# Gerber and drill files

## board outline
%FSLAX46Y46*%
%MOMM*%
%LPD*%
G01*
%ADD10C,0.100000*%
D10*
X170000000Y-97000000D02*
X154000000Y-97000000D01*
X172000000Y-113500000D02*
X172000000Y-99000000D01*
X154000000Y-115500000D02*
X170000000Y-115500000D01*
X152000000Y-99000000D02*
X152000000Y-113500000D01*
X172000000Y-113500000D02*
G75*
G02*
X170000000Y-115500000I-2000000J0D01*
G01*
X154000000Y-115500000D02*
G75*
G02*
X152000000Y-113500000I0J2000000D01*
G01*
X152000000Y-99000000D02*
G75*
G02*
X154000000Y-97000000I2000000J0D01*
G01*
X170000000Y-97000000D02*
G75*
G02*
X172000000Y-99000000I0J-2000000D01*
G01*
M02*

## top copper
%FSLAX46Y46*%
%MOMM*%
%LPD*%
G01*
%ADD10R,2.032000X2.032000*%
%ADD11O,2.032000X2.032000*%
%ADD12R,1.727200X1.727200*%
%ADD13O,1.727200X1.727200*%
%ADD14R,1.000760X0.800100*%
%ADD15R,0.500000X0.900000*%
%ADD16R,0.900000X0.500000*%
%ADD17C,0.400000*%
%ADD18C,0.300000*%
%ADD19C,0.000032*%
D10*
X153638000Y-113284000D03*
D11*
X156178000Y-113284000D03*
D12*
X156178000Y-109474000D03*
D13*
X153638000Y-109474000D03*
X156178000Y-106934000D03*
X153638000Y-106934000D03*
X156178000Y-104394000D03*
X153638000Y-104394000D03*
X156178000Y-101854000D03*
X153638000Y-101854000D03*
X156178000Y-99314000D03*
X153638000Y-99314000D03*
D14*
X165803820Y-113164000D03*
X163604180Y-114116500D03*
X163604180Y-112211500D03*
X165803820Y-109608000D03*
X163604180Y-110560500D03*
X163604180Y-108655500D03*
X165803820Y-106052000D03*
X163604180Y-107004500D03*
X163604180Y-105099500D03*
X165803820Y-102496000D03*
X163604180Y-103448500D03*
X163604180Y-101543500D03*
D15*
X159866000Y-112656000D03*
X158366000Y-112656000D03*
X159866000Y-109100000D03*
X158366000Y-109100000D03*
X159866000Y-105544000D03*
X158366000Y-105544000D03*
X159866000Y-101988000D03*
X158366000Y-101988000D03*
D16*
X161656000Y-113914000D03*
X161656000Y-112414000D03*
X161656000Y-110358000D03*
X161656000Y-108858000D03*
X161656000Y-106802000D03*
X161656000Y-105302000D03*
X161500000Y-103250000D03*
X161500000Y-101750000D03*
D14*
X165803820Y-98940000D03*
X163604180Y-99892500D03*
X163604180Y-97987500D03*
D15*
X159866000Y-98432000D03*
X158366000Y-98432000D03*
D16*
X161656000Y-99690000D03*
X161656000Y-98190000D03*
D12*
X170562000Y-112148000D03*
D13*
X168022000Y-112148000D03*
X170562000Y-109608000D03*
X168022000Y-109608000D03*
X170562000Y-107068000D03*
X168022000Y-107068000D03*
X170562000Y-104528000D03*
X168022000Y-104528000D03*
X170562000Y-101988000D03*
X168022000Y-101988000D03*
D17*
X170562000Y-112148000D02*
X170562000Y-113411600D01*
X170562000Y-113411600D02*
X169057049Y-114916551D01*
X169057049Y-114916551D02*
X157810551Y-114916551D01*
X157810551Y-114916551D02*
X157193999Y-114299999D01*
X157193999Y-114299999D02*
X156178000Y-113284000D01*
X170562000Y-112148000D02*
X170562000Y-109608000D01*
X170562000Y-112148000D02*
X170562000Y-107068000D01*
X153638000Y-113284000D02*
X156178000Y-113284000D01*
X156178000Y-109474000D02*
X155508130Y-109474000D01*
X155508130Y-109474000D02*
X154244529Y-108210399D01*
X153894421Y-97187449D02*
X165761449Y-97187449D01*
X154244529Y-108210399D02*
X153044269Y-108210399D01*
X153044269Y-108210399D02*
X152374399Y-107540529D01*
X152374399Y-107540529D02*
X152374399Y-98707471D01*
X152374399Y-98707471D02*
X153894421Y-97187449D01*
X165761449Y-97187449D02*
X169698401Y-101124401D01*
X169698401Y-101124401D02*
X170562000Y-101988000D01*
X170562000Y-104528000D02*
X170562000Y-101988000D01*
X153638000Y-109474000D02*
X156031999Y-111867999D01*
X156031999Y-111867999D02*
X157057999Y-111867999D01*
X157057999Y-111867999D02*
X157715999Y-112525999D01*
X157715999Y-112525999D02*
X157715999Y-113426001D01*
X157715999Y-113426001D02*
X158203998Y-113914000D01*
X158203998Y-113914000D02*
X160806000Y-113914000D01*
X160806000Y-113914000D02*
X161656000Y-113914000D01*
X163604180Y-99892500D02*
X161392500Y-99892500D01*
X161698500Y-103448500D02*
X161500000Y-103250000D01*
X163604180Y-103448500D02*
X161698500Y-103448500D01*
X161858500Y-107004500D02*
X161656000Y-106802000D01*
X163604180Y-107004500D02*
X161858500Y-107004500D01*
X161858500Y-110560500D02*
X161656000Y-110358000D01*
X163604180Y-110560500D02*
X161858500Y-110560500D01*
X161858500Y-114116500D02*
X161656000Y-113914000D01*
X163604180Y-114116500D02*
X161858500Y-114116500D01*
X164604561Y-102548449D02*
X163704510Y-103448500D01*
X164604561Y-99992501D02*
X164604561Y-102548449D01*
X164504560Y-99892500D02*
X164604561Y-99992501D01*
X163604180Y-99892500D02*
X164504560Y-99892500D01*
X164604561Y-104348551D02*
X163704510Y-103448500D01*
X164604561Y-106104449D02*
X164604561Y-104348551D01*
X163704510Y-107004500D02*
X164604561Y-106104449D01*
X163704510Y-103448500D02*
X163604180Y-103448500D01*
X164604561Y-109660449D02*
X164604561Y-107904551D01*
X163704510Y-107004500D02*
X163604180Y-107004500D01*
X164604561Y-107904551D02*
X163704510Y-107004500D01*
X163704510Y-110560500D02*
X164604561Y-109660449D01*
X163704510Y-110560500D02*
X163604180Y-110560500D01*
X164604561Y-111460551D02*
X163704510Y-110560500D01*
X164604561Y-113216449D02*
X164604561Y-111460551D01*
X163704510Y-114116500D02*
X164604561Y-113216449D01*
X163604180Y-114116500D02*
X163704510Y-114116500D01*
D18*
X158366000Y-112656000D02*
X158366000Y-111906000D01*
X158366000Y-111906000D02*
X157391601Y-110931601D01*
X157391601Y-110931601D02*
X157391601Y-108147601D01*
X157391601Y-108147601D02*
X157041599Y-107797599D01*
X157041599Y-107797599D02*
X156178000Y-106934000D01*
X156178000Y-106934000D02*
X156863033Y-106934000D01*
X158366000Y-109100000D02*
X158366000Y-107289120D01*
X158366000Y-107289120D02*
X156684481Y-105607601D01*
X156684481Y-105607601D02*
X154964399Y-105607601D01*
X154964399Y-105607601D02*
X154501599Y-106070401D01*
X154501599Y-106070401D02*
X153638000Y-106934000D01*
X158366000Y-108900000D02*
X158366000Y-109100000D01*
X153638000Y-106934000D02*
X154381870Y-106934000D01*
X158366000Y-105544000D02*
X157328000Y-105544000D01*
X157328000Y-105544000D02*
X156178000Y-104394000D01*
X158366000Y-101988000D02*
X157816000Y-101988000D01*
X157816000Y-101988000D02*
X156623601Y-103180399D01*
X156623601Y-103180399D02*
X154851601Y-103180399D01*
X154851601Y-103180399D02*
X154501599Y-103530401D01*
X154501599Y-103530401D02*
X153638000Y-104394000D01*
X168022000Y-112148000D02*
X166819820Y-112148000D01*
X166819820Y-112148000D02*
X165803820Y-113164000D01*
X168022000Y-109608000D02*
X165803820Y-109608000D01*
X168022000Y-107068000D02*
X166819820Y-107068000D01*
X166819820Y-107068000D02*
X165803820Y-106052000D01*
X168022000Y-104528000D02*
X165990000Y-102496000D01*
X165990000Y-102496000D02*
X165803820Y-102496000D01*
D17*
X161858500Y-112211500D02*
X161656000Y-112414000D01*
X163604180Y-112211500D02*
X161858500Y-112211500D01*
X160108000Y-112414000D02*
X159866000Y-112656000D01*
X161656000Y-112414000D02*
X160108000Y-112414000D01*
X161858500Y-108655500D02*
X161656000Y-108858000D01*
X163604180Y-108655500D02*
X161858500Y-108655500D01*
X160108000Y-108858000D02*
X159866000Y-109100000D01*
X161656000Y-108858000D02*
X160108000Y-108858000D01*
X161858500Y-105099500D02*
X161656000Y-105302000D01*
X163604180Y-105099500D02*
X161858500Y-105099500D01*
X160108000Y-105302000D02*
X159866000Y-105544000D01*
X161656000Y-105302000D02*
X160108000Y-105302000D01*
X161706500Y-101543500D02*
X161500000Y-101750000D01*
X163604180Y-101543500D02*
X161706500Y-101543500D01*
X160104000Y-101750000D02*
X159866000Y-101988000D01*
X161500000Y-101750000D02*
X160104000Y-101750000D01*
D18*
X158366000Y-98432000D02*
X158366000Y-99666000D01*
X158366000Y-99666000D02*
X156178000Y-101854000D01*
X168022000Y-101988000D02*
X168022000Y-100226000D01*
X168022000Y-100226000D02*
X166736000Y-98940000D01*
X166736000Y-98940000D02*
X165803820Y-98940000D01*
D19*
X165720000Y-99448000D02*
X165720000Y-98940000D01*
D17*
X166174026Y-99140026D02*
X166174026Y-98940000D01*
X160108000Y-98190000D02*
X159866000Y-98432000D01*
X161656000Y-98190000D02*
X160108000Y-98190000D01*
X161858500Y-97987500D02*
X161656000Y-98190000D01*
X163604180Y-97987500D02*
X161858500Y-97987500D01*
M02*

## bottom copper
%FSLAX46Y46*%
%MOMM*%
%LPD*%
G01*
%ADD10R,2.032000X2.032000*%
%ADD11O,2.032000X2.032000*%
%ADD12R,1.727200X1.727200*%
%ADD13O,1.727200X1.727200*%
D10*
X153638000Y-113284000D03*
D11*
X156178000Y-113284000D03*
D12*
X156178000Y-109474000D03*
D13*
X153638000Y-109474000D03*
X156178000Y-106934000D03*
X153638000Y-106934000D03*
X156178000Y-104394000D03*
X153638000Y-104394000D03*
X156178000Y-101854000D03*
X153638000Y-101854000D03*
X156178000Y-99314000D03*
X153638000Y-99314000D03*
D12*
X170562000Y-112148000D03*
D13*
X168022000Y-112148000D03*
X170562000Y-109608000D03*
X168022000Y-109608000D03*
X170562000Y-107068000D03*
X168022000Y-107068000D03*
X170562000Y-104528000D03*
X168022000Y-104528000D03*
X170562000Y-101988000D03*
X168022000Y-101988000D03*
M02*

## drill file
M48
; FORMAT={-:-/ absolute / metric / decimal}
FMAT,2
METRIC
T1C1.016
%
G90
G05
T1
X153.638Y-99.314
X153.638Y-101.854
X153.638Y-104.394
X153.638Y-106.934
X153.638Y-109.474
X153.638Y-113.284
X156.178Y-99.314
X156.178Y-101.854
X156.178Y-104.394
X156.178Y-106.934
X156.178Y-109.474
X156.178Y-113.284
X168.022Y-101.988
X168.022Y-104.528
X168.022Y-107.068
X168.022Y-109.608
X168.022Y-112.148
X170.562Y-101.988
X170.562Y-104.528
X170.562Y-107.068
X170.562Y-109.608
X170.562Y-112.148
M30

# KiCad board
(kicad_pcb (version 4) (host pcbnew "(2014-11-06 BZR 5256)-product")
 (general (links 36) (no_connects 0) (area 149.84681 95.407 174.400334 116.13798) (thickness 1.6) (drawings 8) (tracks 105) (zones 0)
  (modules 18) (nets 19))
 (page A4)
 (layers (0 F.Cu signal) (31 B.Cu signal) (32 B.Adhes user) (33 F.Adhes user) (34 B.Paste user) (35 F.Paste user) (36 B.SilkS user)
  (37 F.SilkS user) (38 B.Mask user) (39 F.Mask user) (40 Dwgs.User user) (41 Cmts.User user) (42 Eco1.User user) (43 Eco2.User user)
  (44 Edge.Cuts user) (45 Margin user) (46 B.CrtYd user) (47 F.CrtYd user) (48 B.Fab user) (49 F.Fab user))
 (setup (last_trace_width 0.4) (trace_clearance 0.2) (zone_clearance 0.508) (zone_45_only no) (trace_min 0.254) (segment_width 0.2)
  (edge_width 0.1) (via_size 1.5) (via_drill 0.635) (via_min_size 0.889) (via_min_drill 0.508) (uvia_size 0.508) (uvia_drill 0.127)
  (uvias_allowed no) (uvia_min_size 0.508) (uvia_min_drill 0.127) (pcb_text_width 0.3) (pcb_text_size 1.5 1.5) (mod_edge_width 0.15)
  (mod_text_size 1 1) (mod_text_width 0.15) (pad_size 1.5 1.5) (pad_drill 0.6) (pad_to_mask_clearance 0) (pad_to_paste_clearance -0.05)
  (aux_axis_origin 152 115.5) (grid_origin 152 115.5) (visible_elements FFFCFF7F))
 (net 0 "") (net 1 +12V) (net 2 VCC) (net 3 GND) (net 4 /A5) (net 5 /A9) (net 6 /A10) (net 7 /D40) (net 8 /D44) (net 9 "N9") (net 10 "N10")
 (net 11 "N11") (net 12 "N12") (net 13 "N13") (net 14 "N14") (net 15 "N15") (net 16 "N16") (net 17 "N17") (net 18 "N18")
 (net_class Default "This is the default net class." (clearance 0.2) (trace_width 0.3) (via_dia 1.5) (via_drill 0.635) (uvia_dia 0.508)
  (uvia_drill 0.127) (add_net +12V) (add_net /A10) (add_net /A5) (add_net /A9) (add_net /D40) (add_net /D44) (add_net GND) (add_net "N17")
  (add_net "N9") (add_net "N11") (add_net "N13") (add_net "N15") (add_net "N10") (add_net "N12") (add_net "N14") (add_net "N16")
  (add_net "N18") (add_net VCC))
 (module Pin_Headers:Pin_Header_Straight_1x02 (layer F.Cu) (at 154.908 113.284)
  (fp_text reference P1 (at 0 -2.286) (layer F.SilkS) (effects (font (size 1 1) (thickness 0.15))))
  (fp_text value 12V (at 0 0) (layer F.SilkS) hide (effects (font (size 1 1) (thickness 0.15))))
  (pad 1 thru_hole rect (at -1.27 0) (size 2.032 2.032) (drill 1.016) (layers *.Cu *.Mask F.SilkS) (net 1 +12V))
  (pad 2 thru_hole oval (at 1.27 0) (size 2.032 2.032) (drill 1.016) (layers *.Cu *.Mask F.SilkS) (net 1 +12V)))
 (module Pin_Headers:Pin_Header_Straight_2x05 (layer F.Cu) (at 154.908 104.394 90)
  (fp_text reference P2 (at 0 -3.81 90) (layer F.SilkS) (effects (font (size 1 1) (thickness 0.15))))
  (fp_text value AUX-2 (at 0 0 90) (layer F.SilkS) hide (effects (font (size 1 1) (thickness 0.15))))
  (pad 1 thru_hole rect (at -5.08 1.27 90) (size 1.7272 1.7272) (drill 1.016) (layers *.Cu *.Mask F.SilkS) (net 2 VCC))
  (pad 2 thru_hole oval (at -5.08 -1.27 90) (size 1.7272 1.7272) (drill 1.016) (layers *.Cu *.Mask F.SilkS) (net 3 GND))
  (pad 3 thru_hole oval (at -2.54 1.27 90) (size 1.7272 1.7272) (drill 1.016) (layers *.Cu *.Mask F.SilkS) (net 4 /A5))
  (pad 4 thru_hole oval (at -2.54 -1.27 90) (size 1.7272 1.7272) (drill 1.016) (layers *.Cu *.Mask F.SilkS) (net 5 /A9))
  (pad 5 thru_hole oval (at 0 1.27 90) (size 1.7272 1.7272) (drill 1.016) (layers *.Cu *.Mask F.SilkS) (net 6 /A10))
  (pad 6 thru_hole oval (at 0 -1.27 90) (size 1.7272 1.7272) (drill 1.016) (layers *.Cu *.Mask F.SilkS) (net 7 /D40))
  (pad 7 thru_hole oval (at 2.54 1.27 90) (size 1.7272 1.7272) (drill 1.016) (layers *.Cu *.Mask F.SilkS) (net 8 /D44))
  (pad 8 thru_hole oval (at 2.54 -1.27 90) (size 1.7272 1.7272) (drill 1.016) (layers *.Cu *.Mask F.SilkS))
  (pad 9 thru_hole oval (at 5.08 1.27 90) (size 1.7272 1.7272) (drill 1.016) (layers *.Cu *.Mask F.SilkS))
  (pad 10 thru_hole oval (at 5.08 -1.27 90) (size 1.7272 1.7272) (drill 1.016) (layers *.Cu *.Mask F.SilkS)))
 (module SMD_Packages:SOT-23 (layer F.Cu) (at 164.704 113.164 270)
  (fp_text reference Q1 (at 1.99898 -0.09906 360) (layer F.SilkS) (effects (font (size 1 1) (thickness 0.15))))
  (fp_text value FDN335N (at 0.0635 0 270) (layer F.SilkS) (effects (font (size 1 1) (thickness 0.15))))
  (pad 3 smd rect (at 0 -1.09982 270) (size 0.8001 1.00076) (layers F.Cu F.Paste F.Mask) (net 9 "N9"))
  (pad 2 smd rect (at 0.9525 1.09982 270) (size 0.8001 1.00076) (layers F.Cu F.Paste F.Mask) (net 3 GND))
  (pad 1 smd rect (at -0.9525 1.09982 270) (size 0.8001 1.00076) (layers F.Cu F.Paste F.Mask) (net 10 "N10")))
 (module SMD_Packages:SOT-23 (layer F.Cu) (at 164.704 109.608 270)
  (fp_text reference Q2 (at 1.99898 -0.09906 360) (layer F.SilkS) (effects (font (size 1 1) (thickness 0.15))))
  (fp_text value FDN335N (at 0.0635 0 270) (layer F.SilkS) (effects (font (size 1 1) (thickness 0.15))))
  (pad 3 smd rect (at 0 -1.09982 270) (size 0.8001 1.00076) (layers F.Cu F.Paste F.Mask) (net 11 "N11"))
  (pad 2 smd rect (at 0.9525 1.09982 270) (size 0.8001 1.00076) (layers F.Cu F.Paste F.Mask) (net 3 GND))
  (pad 1 smd rect (at -0.9525 1.09982 270) (size 0.8001 1.00076) (layers F.Cu F.Paste F.Mask) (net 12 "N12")))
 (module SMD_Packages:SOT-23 (layer F.Cu) (at 164.704 106.052 270)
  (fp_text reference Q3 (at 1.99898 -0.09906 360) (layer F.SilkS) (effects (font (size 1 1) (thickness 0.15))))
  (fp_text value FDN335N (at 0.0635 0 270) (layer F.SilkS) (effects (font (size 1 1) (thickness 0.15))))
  (pad 3 smd rect (at 0 -1.09982 270) (size 0.8001 1.00076) (layers F.Cu F.Paste F.Mask) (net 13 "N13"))
  (pad 2 smd rect (at 0.9525 1.09982 270) (size 0.8001 1.00076) (layers F.Cu F.Paste F.Mask) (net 3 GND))
  (pad 1 smd rect (at -0.9525 1.09982 270) (size 0.8001 1.00076) (layers F.Cu F.Paste F.Mask) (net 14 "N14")))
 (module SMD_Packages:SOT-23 (layer F.Cu) (at 164.704 102.496 270)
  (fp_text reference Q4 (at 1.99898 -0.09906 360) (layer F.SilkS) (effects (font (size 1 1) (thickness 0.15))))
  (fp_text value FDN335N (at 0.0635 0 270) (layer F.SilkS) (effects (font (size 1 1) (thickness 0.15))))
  (pad 3 smd rect (at 0 -1.09982 270) (size 0.8001 1.00076) (layers F.Cu F.Paste F.Mask) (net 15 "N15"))
  (pad 2 smd rect (at 0.9525 1.09982 270) (size 0.8001 1.00076) (layers F.Cu F.Paste F.Mask) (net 3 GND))
  (pad 1 smd rect (at -0.9525 1.09982 270) (size 0.8001 1.00076) (layers F.Cu F.Paste F.Mask) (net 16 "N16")))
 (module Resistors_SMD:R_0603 (layer F.Cu) (at 159.116 112.656 180)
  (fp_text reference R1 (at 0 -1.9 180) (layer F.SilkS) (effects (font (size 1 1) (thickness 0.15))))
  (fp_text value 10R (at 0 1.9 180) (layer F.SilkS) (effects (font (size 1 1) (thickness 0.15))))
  (pad 1 smd rect (at -0.75 0 180) (size 0.5 0.9) (layers F.Cu F.Paste F.Mask) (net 10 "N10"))
  (pad 2 smd rect (at 0.75 0 180) (size 0.5 0.9) (layers F.Cu F.Paste F.Mask) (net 4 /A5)))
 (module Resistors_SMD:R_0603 (layer F.Cu) (at 159.116 109.1 180)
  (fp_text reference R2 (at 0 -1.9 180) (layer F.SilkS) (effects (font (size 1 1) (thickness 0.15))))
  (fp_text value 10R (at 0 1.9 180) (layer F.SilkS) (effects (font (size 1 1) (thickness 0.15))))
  (pad 1 smd rect (at -0.75 0 180) (size 0.5 0.9) (layers F.Cu F.Paste F.Mask) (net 12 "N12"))
  (pad 2 smd rect (at 0.75 0 180) (size 0.5 0.9) (layers F.Cu F.Paste F.Mask) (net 5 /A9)))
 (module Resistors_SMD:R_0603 (layer F.Cu) (at 159.116 105.544 180)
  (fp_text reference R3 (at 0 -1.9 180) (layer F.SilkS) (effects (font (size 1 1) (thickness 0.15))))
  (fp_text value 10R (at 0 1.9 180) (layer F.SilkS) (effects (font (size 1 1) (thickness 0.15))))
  (pad 1 smd rect (at -0.75 0 180) (size 0.5 0.9) (layers F.Cu F.Paste F.Mask) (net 14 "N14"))
  (pad 2 smd rect (at 0.75 0 180) (size 0.5 0.9) (layers F.Cu F.Paste F.Mask) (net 6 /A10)))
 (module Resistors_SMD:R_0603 (layer F.Cu) (at 159.116 101.988 180)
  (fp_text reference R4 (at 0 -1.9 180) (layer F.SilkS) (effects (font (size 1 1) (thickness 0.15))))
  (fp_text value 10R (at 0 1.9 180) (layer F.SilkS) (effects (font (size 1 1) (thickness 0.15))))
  (pad 1 smd rect (at -0.75 0 180) (size 0.5 0.9) (layers F.Cu F.Paste F.Mask) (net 16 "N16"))
  (pad 2 smd rect (at 0.75 0 180) (size 0.5 0.9) (layers F.Cu F.Paste F.Mask) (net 7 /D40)))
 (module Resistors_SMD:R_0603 (layer F.Cu) (at 161.656 113.164 90)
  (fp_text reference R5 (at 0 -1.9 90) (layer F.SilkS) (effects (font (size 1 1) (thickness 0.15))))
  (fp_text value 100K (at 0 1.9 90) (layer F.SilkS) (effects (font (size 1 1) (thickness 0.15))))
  (pad 1 smd rect (at -0.75 0 90) (size 0.5 0.9) (layers F.Cu F.Paste F.Mask) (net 3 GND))
  (pad 2 smd rect (at 0.75 0 90) (size 0.5 0.9) (layers F.Cu F.Paste F.Mask) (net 10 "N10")))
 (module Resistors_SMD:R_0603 (layer F.Cu) (at 161.656 109.608 90)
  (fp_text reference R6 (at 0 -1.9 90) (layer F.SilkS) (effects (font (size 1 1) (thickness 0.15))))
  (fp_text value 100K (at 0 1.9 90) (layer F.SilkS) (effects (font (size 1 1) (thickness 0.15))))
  (pad 1 smd rect (at -0.75 0 90) (size 0.5 0.9) (layers F.Cu F.Paste F.Mask) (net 3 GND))
  (pad 2 smd rect (at 0.75 0 90) (size 0.5 0.9) (layers F.Cu F.Paste F.Mask) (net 12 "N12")))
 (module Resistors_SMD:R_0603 (layer F.Cu) (at 161.656 106.052 90)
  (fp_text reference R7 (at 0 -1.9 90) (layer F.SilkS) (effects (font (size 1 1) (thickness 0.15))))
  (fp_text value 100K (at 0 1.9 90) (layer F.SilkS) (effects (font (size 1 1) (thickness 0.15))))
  (pad 1 smd rect (at -0.75 0 90) (size 0.5 0.9) (layers F.Cu F.Paste F.Mask) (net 3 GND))
  (pad 2 smd rect (at 0.75 0 90) (size 0.5 0.9) (layers F.Cu F.Paste F.Mask) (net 14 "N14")))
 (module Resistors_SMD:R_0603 (layer F.Cu) (at 161.5 102.5 90)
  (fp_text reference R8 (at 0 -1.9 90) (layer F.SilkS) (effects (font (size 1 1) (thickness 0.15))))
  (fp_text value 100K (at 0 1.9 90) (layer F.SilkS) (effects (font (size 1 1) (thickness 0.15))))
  (pad 1 smd rect (at -0.75 0 90) (size 0.5 0.9) (layers F.Cu F.Paste F.Mask) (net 3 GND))
  (pad 2 smd rect (at 0.75 0 90) (size 0.5 0.9) (layers F.Cu F.Paste F.Mask) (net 16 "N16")))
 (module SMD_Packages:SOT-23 (layer F.Cu) (at 164.704 98.94 270)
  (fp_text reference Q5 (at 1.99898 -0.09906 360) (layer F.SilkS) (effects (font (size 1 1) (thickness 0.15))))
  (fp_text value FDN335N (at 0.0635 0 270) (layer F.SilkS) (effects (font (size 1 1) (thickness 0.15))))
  (pad 3 smd rect (at 0 -1.09982 270) (size 0.8001 1.00076) (layers F.Cu F.Paste F.Mask) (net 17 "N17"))
  (pad 2 smd rect (at 0.9525 1.09982 270) (size 0.8001 1.00076) (layers F.Cu F.Paste F.Mask) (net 3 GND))
  (pad 1 smd rect (at -0.9525 1.09982 270) (size 0.8001 1.00076) (layers F.Cu F.Paste F.Mask) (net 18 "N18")))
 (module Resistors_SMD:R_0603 (layer F.Cu) (at 159.116 98.432 180)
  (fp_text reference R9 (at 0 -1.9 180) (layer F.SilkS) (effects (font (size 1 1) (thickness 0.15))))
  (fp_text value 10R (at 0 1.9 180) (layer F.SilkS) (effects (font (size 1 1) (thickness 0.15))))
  (pad 1 smd rect (at -0.75 0 180) (size 0.5 0.9) (layers F.Cu F.Paste F.Mask) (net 18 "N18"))
  (pad 2 smd rect (at 0.75 0 180) (size 0.5 0.9) (layers F.Cu F.Paste F.Mask) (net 8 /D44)))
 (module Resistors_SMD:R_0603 (layer F.Cu) (at 161.656 98.94 90)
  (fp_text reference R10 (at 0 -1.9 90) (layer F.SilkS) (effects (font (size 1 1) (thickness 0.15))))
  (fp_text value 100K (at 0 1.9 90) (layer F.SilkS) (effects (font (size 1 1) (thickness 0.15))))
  (pad 1 smd rect (at -0.75 0 90) (size 0.5 0.9) (layers F.Cu F.Paste F.Mask) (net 3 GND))
  (pad 2 smd rect (at 0.75 0 90) (size 0.5 0.9) (layers F.Cu F.Paste F.Mask) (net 18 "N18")))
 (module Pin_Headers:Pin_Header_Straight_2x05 (layer F.Cu) (at 169.292 107.068 90)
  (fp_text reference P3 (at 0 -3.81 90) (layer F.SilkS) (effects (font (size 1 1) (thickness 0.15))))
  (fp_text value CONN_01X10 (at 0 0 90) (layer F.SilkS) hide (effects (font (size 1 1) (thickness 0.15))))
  (pad 1 thru_hole rect (at -5.08 1.27 90) (size 1.7272 1.7272) (drill 1.016) (layers *.Cu *.Mask F.SilkS) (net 1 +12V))
  (pad 2 thru_hole oval (at -5.08 -1.27 90) (size 1.7272 1.7272) (drill 1.016) (layers *.Cu *.Mask F.SilkS) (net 9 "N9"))
  (pad 3 thru_hole oval (at -2.54 1.27 90) (size 1.7272 1.7272) (drill 1.016) (layers *.Cu *.Mask F.SilkS) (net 1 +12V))
  (pad 4 thru_hole oval (at -2.54 -1.27 90) (size 1.7272 1.7272) (drill 1.016) (layers *.Cu *.Mask F.SilkS) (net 11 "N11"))
  (pad 5 thru_hole oval (at 0 1.27 90) (size 1.7272 1.7272) (drill 1.016) (layers *.Cu *.Mask F.SilkS) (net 1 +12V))
  (pad 6 thru_hole oval (at 0 -1.27 90) (size 1.7272 1.7272) (drill 1.016) (layers *.Cu *.Mask F.SilkS) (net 13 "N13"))
  (pad 7 thru_hole oval (at 2.54 1.27 90) (size 1.7272 1.7272) (drill 1.016) (layers *.Cu *.Mask F.SilkS) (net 2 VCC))
  (pad 8 thru_hole oval (at 2.54 -1.27 90) (size 1.7272 1.7272) (drill 1.016) (layers *.Cu *.Mask F.SilkS) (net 15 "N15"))
  (pad 9 thru_hole oval (at 5.08 1.27 90) (size 1.7272 1.7272) (drill 1.016) (layers *.Cu *.Mask F.SilkS) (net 2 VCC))
  (pad 10 thru_hole oval (at 5.08 -1.27 90) (size 1.7272 1.7272) (drill 1.016) (layers *.Cu *.Mask F.SilkS) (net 17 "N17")))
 (gr_line (start 170 97) (end 154 97) (angle 90) (layer Edge.Cuts) (width 0.1))
 (gr_line (start 172 113.5) (end 172 99) (angle 90) (layer Edge.Cuts) (width 0.1))
 (gr_line (start 154 115.5) (end 170 115.5) (angle 90) (layer Edge.Cuts) (width 0.1))
 (gr_line (start 152 99) (end 152 113.5) (angle 90) (layer Edge.Cuts) (width 0.1))
 (gr_arc (start 170 113.5) (end 172 113.5) (angle 90) (layer Edge.Cuts) (width 0.1))
 (gr_arc (start 154 113.5) (end 154 115.5) (angle 90) (layer Edge.Cuts) (width 0.1))
 (gr_arc (start 154 99) (end 152 99) (angle 90) (layer Edge.Cuts) (width 0.1))
 (gr_arc (start 170 99) (end 170 97) (angle 90) (layer Edge.Cuts) (width 0.1))
 (segment (start 170.562 112.148) (end 170.562 113.4116) (width 0.4) (layer F.Cu) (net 1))
 (segment (start 170.562 113.4116) (end 169.057049 114.916551) (width 0.4) (layer F.Cu) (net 1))
 (segment (start 169.057049 114.916551) (end 157.810551 114.916551) (width 0.4) (layer F.Cu) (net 1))
 (segment (start 157.810551 114.916551) (end 157.193999 114.299999) (width 0.4) (layer F.Cu) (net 1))
 (segment (start 157.193999 114.299999) (end 156.178 113.284) (width 0.4) (layer F.Cu) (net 1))
 (segment (start 170.562 112.148) (end 170.562 109.608) (width 0.4) (layer F.Cu) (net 1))
 (segment (start 170.562 112.148) (end 170.562 107.068) (width 0.4) (layer F.Cu) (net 1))
 (segment (start 153.638 113.284) (end 156.178 113.284) (width 0.4) (layer F.Cu) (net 1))
 (segment (start 156.178 109.474) (end 155.50813 109.474) (width 0.4) (layer F.Cu) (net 2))
 (segment (start 155.50813 109.474) (end 154.244529 108.210399) (width 0.4) (layer F.Cu) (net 2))
 (segment (start 153.894421 97.187449) (end 165.761449 97.187449) (width 0.4) (layer F.Cu) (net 2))
 (segment (start 154.244529 108.210399) (end 153.044269 108.210399) (width 0.4) (layer F.Cu) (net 2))
 (segment (start 153.044269 108.210399) (end 152.374399 107.540529) (width 0.4) (layer F.Cu) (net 2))
 (segment (start 152.374399 107.540529) (end 152.374399 98.707471) (width 0.4) (layer F.Cu) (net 2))
 (segment (start 152.374399 98.707471) (end 153.894421 97.187449) (width 0.4) (layer F.Cu) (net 2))
 (segment (start 165.761449 97.187449) (end 169.698401 101.124401) (width 0.4) (layer F.Cu) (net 2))
 (segment (start 169.698401 101.124401) (end 170.562 101.988) (width 0.4) (layer F.Cu) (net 2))
 (segment (start 170.562 104.528) (end 170.562 101.988) (width 0.4) (layer F.Cu) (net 2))
 (segment (start 153.638 109.474) (end 156.031999 111.867999) (width 0.4) (layer F.Cu) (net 3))
 (segment (start 156.031999 111.867999) (end 157.057999 111.867999) (width 0.4) (layer F.Cu) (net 3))
 (segment (start 157.057999 111.867999) (end 157.715999 112.525999) (width 0.4) (layer F.Cu) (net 3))
 (segment (start 157.715999 112.525999) (end 157.715999 113.426001) (width 0.4) (layer F.Cu) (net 3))
 (segment (start 157.715999 113.426001) (end 158.203998 113.914) (width 0.4) (layer F.Cu) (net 3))
 (segment (start 158.203998 113.914) (end 160.806 113.914) (width 0.4) (layer F.Cu) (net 3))
 (segment (start 160.806 113.914) (end 161.656 113.914) (width 0.4) (layer F.Cu) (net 3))
 (segment (start 163.60418 99.8925) (end 161.3925 99.8925) (width 0.4) (layer F.Cu) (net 3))
 (segment (start 161.6985 103.4485) (end 161.5 103.25) (width 0.4) (layer F.Cu) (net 3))
 (segment (start 163.60418 103.4485) (end 161.6985 103.4485) (width 0.4) (layer F.Cu) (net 3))
 (segment (start 161.8585 107.0045) (end 161.656 106.802) (width 0.4) (layer F.Cu) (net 3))
 (segment (start 163.60418 107.0045) (end 161.8585 107.0045) (width 0.4) (layer F.Cu) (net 3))
 (segment (start 161.8585 110.5605) (end 161.656 110.358) (width 0.4) (layer F.Cu) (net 3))
 (segment (start 163.60418 110.5605) (end 161.8585 110.5605) (width 0.4) (layer F.Cu) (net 3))
 (segment (start 161.8585 114.1165) (end 161.656 113.914) (width 0.4) (layer F.Cu) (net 3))
 (segment (start 163.60418 114.1165) (end 161.8585 114.1165) (width 0.4) (layer F.Cu) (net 3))
 (segment (start 164.604561 102.548449) (end 163.70451 103.4485) (width 0.4) (layer F.Cu) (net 3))
 (segment (start 164.604561 99.992501) (end 164.604561 102.548449) (width 0.4) (layer F.Cu) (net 3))
 (segment (start 164.50456 99.8925) (end 164.604561 99.992501) (width 0.4) (layer F.Cu) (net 3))
 (segment (start 163.60418 99.8925) (end 164.50456 99.8925) (width 0.4) (layer F.Cu) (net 3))
 (segment (start 164.604561 104.348551) (end 163.70451 103.4485) (width 0.4) (layer F.Cu) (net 3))
 (segment (start 164.604561 106.104449) (end 164.604561 104.348551) (width 0.4) (layer F.Cu) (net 3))
 (segment (start 163.70451 107.0045) (end 164.604561 106.104449) (width 0.4) (layer F.Cu) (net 3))
 (segment (start 163.70451 103.4485) (end 163.60418 103.4485) (width 0.4) (layer F.Cu) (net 3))
 (segment (start 164.604561 109.660449) (end 164.604561 107.904551) (width 0.4) (layer F.Cu) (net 3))
 (segment (start 163.70451 107.0045) (end 163.60418 107.0045) (width 0.4) (layer F.Cu) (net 3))
 (segment (start 164.604561 107.904551) (end 163.70451 107.0045) (width 0.4) (layer F.Cu) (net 3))
 (segment (start 163.70451 110.5605) (end 164.604561 109.660449) (width 0.4) (layer F.Cu) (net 3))
 (segment (start 163.70451 110.5605) (end 163.60418 110.5605) (width 0.4) (layer F.Cu) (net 3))
 (segment (start 164.604561 111.460551) (end 163.70451 110.5605) (width 0.4) (layer F.Cu) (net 3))
 (segment (start 164.604561 113.216449) (end 164.604561 111.460551) (width 0.4) (layer F.Cu) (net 3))
 (segment (start 163.70451 114.1165) (end 164.604561 113.216449) (width 0.4) (layer F.Cu) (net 3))
 (segment (start 163.60418 114.1165) (end 163.70451 114.1165) (width 0.4) (layer F.Cu) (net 3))
 (segment (start 158.366 112.656) (end 158.366 111.906) (width 0.3) (layer F.Cu) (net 4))
 (segment (start 158.366 111.906) (end 157.391601 110.931601) (width 0.3) (layer F.Cu) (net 4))
 (segment (start 157.391601 110.931601) (end 157.391601 108.147601) (width 0.3) (layer F.Cu) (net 4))
 (segment (start 157.391601 108.147601) (end 157.041599 107.797599) (width 0.3) (layer F.Cu) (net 4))
 (segment (start 157.041599 107.797599) (end 156.178 106.934) (width 0.3) (layer F.Cu) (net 4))
 (segment (start 156.178 106.934) (end 156.863033 106.934) (width 0.3) (layer F.Cu) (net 4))
 (segment (start 158.366 109.1) (end 158.366 107.28912) (width 0.3) (layer F.Cu) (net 5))
 (segment (start 158.366 107.28912) (end 156.684481 105.607601) (width 0.3) (layer F.Cu) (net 5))
 (segment (start 156.684481 105.607601) (end 154.964399 105.607601) (width 0.3) (layer F.Cu) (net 5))
 (segment (start 154.964399 105.607601) (end 154.501599 106.070401) (width 0.3) (layer F.Cu) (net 5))
 (segment (start 154.501599 106.070401) (end 153.638 106.934) (width 0.3) (layer F.Cu) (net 5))
 (segment (start 158.366 108.9) (end 158.366 109.1) (width 0.3) (layer F.Cu) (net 5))
 (segment (start 153.638 106.934) (end 154.38187 106.934) (width 0.3) (layer F.Cu) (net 5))
 (segment (start 158.366 105.544) (end 157.328 105.544) (width 0.3) (layer F.Cu) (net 6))
 (segment (start 157.328 105.544) (end 156.178 104.394) (width 0.3) (layer F.Cu) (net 6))
 (segment (start 158.366 101.988) (end 157.816 101.988) (width 0.3) (layer F.Cu) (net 7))
 (segment (start 157.816 101.988) (end 156.623601 103.180399) (width 0.3) (layer F.Cu) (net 7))
 (segment (start 156.623601 103.180399) (end 154.851601 103.180399) (width 0.3) (layer F.Cu) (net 7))
 (segment (start 154.851601 103.180399) (end 154.501599 103.530401) (width 0.3) (layer F.Cu) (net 7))
 (segment (start 154.501599 103.530401) (end 153.638 104.394) (width 0.3) (layer F.Cu) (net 7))
 (segment (start 168.022 112.148) (end 166.81982 112.148) (width 0.3) (layer F.Cu) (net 9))
 (segment (start 166.81982 112.148) (end 165.80382 113.164) (width 0.3) (layer F.Cu) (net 9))
 (segment (start 168.022 109.608) (end 165.80382 109.608) (width 0.3) (layer F.Cu) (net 11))
 (segment (start 168.022 107.068) (end 166.81982 107.068) (width 0.3) (layer F.Cu) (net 13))
 (segment (start 166.81982 107.068) (end 165.80382 106.052) (width 0.3) (layer F.Cu) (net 13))
 (segment (start 168.022 104.528) (end 165.99 102.496) (width 0.3) (layer F.Cu) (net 15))
 (segment (start 165.99 102.496) (end 165.80382 102.496) (width 0.3) (layer F.Cu) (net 15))
 (segment (start 161.8585 112.2115) (end 161.656 112.414) (width 0.4) (layer F.Cu) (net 10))
 (segment (start 163.60418 112.2115) (end 161.8585 112.2115) (width 0.4) (layer F.Cu) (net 10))
 (segment (start 160.108 112.414) (end 159.866 112.656) (width 0.4) (layer F.Cu) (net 10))
 (segment (start 161.656 112.414) (end 160.108 112.414) (width 0.4) (layer F.Cu) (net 10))
 (segment (start 161.8585 108.6555) (end 161.656 108.858) (width 0.4) (layer F.Cu) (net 12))
 (segment (start 163.60418 108.6555) (end 161.8585 108.6555) (width 0.4) (layer F.Cu) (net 12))
 (segment (start 160.108 108.858) (end 159.866 109.1) (width 0.4) (layer F.Cu) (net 12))
 (segment (start 161.656 108.858) (end 160.108 108.858) (width 0.4) (layer F.Cu) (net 12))
 (segment (start 161.8585 105.0995) (end 161.656 105.302) (width 0.4) (layer F.Cu) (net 14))
 (segment (start 163.60418 105.0995) (end 161.8585 105.0995) (width 0.4) (layer F.Cu) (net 14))
 (segment (start 160.108 105.302) (end 159.866 105.544) (width 0.4) (layer F.Cu) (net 14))
 (segment (start 161.656 105.302) (end 160.108 105.302) (width 0.4) (layer F.Cu) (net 14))
 (segment (start 161.7065 101.5435) (end 161.5 101.75) (width 0.4) (layer F.Cu) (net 16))
 (segment (start 163.60418 101.5435) (end 161.7065 101.5435) (width 0.4) (layer F.Cu) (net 16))
 (segment (start 160.104 101.75) (end 159.866 101.988) (width 0.4) (layer F.Cu) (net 16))
 (segment (start 161.5 101.75) (end 160.104 101.75) (width 0.4) (layer F.Cu) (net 16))
 (segment (start 158.366 98.432) (end 158.366 99.666) (width 0.3) (layer F.Cu) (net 8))
 (segment (start 158.366 99.666) (end 156.178 101.854) (width 0.3) (layer F.Cu) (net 8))
 (segment (start 168.022 101.988) (end 168.022 100.226) (width 0.3) (layer F.Cu) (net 17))
 (segment (start 168.022 100.226) (end 166.736 98.94) (width 0.3) (layer F.Cu) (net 17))
 (segment (start 166.736 98.94) (end 165.80382 98.94) (width 0.3) (layer F.Cu) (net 17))
 (segment (start 165.72 99.448) (end 165.72 98.94) (width 0.000032) (layer F.Cu) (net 17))
 (segment (start 166.174026 99.140026) (end 166.174026 98.94) (width 0.4) (layer F.Cu) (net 17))
 (segment (start 160.108 98.19) (end 159.866 98.432) (width 0.4) (layer F.Cu) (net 18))
 (segment (start 161.656 98.19) (end 160.108 98.19) (width 0.4) (layer F.Cu) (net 18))
 (segment (start 161.8585 97.9875) (end 161.656 98.19) (width 0.4) (layer F.Cu) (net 18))
 (segment (start 163.60418 97.9875) (end 161.8585 97.9875) (width 0.4) (layer F.Cu) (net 18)))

